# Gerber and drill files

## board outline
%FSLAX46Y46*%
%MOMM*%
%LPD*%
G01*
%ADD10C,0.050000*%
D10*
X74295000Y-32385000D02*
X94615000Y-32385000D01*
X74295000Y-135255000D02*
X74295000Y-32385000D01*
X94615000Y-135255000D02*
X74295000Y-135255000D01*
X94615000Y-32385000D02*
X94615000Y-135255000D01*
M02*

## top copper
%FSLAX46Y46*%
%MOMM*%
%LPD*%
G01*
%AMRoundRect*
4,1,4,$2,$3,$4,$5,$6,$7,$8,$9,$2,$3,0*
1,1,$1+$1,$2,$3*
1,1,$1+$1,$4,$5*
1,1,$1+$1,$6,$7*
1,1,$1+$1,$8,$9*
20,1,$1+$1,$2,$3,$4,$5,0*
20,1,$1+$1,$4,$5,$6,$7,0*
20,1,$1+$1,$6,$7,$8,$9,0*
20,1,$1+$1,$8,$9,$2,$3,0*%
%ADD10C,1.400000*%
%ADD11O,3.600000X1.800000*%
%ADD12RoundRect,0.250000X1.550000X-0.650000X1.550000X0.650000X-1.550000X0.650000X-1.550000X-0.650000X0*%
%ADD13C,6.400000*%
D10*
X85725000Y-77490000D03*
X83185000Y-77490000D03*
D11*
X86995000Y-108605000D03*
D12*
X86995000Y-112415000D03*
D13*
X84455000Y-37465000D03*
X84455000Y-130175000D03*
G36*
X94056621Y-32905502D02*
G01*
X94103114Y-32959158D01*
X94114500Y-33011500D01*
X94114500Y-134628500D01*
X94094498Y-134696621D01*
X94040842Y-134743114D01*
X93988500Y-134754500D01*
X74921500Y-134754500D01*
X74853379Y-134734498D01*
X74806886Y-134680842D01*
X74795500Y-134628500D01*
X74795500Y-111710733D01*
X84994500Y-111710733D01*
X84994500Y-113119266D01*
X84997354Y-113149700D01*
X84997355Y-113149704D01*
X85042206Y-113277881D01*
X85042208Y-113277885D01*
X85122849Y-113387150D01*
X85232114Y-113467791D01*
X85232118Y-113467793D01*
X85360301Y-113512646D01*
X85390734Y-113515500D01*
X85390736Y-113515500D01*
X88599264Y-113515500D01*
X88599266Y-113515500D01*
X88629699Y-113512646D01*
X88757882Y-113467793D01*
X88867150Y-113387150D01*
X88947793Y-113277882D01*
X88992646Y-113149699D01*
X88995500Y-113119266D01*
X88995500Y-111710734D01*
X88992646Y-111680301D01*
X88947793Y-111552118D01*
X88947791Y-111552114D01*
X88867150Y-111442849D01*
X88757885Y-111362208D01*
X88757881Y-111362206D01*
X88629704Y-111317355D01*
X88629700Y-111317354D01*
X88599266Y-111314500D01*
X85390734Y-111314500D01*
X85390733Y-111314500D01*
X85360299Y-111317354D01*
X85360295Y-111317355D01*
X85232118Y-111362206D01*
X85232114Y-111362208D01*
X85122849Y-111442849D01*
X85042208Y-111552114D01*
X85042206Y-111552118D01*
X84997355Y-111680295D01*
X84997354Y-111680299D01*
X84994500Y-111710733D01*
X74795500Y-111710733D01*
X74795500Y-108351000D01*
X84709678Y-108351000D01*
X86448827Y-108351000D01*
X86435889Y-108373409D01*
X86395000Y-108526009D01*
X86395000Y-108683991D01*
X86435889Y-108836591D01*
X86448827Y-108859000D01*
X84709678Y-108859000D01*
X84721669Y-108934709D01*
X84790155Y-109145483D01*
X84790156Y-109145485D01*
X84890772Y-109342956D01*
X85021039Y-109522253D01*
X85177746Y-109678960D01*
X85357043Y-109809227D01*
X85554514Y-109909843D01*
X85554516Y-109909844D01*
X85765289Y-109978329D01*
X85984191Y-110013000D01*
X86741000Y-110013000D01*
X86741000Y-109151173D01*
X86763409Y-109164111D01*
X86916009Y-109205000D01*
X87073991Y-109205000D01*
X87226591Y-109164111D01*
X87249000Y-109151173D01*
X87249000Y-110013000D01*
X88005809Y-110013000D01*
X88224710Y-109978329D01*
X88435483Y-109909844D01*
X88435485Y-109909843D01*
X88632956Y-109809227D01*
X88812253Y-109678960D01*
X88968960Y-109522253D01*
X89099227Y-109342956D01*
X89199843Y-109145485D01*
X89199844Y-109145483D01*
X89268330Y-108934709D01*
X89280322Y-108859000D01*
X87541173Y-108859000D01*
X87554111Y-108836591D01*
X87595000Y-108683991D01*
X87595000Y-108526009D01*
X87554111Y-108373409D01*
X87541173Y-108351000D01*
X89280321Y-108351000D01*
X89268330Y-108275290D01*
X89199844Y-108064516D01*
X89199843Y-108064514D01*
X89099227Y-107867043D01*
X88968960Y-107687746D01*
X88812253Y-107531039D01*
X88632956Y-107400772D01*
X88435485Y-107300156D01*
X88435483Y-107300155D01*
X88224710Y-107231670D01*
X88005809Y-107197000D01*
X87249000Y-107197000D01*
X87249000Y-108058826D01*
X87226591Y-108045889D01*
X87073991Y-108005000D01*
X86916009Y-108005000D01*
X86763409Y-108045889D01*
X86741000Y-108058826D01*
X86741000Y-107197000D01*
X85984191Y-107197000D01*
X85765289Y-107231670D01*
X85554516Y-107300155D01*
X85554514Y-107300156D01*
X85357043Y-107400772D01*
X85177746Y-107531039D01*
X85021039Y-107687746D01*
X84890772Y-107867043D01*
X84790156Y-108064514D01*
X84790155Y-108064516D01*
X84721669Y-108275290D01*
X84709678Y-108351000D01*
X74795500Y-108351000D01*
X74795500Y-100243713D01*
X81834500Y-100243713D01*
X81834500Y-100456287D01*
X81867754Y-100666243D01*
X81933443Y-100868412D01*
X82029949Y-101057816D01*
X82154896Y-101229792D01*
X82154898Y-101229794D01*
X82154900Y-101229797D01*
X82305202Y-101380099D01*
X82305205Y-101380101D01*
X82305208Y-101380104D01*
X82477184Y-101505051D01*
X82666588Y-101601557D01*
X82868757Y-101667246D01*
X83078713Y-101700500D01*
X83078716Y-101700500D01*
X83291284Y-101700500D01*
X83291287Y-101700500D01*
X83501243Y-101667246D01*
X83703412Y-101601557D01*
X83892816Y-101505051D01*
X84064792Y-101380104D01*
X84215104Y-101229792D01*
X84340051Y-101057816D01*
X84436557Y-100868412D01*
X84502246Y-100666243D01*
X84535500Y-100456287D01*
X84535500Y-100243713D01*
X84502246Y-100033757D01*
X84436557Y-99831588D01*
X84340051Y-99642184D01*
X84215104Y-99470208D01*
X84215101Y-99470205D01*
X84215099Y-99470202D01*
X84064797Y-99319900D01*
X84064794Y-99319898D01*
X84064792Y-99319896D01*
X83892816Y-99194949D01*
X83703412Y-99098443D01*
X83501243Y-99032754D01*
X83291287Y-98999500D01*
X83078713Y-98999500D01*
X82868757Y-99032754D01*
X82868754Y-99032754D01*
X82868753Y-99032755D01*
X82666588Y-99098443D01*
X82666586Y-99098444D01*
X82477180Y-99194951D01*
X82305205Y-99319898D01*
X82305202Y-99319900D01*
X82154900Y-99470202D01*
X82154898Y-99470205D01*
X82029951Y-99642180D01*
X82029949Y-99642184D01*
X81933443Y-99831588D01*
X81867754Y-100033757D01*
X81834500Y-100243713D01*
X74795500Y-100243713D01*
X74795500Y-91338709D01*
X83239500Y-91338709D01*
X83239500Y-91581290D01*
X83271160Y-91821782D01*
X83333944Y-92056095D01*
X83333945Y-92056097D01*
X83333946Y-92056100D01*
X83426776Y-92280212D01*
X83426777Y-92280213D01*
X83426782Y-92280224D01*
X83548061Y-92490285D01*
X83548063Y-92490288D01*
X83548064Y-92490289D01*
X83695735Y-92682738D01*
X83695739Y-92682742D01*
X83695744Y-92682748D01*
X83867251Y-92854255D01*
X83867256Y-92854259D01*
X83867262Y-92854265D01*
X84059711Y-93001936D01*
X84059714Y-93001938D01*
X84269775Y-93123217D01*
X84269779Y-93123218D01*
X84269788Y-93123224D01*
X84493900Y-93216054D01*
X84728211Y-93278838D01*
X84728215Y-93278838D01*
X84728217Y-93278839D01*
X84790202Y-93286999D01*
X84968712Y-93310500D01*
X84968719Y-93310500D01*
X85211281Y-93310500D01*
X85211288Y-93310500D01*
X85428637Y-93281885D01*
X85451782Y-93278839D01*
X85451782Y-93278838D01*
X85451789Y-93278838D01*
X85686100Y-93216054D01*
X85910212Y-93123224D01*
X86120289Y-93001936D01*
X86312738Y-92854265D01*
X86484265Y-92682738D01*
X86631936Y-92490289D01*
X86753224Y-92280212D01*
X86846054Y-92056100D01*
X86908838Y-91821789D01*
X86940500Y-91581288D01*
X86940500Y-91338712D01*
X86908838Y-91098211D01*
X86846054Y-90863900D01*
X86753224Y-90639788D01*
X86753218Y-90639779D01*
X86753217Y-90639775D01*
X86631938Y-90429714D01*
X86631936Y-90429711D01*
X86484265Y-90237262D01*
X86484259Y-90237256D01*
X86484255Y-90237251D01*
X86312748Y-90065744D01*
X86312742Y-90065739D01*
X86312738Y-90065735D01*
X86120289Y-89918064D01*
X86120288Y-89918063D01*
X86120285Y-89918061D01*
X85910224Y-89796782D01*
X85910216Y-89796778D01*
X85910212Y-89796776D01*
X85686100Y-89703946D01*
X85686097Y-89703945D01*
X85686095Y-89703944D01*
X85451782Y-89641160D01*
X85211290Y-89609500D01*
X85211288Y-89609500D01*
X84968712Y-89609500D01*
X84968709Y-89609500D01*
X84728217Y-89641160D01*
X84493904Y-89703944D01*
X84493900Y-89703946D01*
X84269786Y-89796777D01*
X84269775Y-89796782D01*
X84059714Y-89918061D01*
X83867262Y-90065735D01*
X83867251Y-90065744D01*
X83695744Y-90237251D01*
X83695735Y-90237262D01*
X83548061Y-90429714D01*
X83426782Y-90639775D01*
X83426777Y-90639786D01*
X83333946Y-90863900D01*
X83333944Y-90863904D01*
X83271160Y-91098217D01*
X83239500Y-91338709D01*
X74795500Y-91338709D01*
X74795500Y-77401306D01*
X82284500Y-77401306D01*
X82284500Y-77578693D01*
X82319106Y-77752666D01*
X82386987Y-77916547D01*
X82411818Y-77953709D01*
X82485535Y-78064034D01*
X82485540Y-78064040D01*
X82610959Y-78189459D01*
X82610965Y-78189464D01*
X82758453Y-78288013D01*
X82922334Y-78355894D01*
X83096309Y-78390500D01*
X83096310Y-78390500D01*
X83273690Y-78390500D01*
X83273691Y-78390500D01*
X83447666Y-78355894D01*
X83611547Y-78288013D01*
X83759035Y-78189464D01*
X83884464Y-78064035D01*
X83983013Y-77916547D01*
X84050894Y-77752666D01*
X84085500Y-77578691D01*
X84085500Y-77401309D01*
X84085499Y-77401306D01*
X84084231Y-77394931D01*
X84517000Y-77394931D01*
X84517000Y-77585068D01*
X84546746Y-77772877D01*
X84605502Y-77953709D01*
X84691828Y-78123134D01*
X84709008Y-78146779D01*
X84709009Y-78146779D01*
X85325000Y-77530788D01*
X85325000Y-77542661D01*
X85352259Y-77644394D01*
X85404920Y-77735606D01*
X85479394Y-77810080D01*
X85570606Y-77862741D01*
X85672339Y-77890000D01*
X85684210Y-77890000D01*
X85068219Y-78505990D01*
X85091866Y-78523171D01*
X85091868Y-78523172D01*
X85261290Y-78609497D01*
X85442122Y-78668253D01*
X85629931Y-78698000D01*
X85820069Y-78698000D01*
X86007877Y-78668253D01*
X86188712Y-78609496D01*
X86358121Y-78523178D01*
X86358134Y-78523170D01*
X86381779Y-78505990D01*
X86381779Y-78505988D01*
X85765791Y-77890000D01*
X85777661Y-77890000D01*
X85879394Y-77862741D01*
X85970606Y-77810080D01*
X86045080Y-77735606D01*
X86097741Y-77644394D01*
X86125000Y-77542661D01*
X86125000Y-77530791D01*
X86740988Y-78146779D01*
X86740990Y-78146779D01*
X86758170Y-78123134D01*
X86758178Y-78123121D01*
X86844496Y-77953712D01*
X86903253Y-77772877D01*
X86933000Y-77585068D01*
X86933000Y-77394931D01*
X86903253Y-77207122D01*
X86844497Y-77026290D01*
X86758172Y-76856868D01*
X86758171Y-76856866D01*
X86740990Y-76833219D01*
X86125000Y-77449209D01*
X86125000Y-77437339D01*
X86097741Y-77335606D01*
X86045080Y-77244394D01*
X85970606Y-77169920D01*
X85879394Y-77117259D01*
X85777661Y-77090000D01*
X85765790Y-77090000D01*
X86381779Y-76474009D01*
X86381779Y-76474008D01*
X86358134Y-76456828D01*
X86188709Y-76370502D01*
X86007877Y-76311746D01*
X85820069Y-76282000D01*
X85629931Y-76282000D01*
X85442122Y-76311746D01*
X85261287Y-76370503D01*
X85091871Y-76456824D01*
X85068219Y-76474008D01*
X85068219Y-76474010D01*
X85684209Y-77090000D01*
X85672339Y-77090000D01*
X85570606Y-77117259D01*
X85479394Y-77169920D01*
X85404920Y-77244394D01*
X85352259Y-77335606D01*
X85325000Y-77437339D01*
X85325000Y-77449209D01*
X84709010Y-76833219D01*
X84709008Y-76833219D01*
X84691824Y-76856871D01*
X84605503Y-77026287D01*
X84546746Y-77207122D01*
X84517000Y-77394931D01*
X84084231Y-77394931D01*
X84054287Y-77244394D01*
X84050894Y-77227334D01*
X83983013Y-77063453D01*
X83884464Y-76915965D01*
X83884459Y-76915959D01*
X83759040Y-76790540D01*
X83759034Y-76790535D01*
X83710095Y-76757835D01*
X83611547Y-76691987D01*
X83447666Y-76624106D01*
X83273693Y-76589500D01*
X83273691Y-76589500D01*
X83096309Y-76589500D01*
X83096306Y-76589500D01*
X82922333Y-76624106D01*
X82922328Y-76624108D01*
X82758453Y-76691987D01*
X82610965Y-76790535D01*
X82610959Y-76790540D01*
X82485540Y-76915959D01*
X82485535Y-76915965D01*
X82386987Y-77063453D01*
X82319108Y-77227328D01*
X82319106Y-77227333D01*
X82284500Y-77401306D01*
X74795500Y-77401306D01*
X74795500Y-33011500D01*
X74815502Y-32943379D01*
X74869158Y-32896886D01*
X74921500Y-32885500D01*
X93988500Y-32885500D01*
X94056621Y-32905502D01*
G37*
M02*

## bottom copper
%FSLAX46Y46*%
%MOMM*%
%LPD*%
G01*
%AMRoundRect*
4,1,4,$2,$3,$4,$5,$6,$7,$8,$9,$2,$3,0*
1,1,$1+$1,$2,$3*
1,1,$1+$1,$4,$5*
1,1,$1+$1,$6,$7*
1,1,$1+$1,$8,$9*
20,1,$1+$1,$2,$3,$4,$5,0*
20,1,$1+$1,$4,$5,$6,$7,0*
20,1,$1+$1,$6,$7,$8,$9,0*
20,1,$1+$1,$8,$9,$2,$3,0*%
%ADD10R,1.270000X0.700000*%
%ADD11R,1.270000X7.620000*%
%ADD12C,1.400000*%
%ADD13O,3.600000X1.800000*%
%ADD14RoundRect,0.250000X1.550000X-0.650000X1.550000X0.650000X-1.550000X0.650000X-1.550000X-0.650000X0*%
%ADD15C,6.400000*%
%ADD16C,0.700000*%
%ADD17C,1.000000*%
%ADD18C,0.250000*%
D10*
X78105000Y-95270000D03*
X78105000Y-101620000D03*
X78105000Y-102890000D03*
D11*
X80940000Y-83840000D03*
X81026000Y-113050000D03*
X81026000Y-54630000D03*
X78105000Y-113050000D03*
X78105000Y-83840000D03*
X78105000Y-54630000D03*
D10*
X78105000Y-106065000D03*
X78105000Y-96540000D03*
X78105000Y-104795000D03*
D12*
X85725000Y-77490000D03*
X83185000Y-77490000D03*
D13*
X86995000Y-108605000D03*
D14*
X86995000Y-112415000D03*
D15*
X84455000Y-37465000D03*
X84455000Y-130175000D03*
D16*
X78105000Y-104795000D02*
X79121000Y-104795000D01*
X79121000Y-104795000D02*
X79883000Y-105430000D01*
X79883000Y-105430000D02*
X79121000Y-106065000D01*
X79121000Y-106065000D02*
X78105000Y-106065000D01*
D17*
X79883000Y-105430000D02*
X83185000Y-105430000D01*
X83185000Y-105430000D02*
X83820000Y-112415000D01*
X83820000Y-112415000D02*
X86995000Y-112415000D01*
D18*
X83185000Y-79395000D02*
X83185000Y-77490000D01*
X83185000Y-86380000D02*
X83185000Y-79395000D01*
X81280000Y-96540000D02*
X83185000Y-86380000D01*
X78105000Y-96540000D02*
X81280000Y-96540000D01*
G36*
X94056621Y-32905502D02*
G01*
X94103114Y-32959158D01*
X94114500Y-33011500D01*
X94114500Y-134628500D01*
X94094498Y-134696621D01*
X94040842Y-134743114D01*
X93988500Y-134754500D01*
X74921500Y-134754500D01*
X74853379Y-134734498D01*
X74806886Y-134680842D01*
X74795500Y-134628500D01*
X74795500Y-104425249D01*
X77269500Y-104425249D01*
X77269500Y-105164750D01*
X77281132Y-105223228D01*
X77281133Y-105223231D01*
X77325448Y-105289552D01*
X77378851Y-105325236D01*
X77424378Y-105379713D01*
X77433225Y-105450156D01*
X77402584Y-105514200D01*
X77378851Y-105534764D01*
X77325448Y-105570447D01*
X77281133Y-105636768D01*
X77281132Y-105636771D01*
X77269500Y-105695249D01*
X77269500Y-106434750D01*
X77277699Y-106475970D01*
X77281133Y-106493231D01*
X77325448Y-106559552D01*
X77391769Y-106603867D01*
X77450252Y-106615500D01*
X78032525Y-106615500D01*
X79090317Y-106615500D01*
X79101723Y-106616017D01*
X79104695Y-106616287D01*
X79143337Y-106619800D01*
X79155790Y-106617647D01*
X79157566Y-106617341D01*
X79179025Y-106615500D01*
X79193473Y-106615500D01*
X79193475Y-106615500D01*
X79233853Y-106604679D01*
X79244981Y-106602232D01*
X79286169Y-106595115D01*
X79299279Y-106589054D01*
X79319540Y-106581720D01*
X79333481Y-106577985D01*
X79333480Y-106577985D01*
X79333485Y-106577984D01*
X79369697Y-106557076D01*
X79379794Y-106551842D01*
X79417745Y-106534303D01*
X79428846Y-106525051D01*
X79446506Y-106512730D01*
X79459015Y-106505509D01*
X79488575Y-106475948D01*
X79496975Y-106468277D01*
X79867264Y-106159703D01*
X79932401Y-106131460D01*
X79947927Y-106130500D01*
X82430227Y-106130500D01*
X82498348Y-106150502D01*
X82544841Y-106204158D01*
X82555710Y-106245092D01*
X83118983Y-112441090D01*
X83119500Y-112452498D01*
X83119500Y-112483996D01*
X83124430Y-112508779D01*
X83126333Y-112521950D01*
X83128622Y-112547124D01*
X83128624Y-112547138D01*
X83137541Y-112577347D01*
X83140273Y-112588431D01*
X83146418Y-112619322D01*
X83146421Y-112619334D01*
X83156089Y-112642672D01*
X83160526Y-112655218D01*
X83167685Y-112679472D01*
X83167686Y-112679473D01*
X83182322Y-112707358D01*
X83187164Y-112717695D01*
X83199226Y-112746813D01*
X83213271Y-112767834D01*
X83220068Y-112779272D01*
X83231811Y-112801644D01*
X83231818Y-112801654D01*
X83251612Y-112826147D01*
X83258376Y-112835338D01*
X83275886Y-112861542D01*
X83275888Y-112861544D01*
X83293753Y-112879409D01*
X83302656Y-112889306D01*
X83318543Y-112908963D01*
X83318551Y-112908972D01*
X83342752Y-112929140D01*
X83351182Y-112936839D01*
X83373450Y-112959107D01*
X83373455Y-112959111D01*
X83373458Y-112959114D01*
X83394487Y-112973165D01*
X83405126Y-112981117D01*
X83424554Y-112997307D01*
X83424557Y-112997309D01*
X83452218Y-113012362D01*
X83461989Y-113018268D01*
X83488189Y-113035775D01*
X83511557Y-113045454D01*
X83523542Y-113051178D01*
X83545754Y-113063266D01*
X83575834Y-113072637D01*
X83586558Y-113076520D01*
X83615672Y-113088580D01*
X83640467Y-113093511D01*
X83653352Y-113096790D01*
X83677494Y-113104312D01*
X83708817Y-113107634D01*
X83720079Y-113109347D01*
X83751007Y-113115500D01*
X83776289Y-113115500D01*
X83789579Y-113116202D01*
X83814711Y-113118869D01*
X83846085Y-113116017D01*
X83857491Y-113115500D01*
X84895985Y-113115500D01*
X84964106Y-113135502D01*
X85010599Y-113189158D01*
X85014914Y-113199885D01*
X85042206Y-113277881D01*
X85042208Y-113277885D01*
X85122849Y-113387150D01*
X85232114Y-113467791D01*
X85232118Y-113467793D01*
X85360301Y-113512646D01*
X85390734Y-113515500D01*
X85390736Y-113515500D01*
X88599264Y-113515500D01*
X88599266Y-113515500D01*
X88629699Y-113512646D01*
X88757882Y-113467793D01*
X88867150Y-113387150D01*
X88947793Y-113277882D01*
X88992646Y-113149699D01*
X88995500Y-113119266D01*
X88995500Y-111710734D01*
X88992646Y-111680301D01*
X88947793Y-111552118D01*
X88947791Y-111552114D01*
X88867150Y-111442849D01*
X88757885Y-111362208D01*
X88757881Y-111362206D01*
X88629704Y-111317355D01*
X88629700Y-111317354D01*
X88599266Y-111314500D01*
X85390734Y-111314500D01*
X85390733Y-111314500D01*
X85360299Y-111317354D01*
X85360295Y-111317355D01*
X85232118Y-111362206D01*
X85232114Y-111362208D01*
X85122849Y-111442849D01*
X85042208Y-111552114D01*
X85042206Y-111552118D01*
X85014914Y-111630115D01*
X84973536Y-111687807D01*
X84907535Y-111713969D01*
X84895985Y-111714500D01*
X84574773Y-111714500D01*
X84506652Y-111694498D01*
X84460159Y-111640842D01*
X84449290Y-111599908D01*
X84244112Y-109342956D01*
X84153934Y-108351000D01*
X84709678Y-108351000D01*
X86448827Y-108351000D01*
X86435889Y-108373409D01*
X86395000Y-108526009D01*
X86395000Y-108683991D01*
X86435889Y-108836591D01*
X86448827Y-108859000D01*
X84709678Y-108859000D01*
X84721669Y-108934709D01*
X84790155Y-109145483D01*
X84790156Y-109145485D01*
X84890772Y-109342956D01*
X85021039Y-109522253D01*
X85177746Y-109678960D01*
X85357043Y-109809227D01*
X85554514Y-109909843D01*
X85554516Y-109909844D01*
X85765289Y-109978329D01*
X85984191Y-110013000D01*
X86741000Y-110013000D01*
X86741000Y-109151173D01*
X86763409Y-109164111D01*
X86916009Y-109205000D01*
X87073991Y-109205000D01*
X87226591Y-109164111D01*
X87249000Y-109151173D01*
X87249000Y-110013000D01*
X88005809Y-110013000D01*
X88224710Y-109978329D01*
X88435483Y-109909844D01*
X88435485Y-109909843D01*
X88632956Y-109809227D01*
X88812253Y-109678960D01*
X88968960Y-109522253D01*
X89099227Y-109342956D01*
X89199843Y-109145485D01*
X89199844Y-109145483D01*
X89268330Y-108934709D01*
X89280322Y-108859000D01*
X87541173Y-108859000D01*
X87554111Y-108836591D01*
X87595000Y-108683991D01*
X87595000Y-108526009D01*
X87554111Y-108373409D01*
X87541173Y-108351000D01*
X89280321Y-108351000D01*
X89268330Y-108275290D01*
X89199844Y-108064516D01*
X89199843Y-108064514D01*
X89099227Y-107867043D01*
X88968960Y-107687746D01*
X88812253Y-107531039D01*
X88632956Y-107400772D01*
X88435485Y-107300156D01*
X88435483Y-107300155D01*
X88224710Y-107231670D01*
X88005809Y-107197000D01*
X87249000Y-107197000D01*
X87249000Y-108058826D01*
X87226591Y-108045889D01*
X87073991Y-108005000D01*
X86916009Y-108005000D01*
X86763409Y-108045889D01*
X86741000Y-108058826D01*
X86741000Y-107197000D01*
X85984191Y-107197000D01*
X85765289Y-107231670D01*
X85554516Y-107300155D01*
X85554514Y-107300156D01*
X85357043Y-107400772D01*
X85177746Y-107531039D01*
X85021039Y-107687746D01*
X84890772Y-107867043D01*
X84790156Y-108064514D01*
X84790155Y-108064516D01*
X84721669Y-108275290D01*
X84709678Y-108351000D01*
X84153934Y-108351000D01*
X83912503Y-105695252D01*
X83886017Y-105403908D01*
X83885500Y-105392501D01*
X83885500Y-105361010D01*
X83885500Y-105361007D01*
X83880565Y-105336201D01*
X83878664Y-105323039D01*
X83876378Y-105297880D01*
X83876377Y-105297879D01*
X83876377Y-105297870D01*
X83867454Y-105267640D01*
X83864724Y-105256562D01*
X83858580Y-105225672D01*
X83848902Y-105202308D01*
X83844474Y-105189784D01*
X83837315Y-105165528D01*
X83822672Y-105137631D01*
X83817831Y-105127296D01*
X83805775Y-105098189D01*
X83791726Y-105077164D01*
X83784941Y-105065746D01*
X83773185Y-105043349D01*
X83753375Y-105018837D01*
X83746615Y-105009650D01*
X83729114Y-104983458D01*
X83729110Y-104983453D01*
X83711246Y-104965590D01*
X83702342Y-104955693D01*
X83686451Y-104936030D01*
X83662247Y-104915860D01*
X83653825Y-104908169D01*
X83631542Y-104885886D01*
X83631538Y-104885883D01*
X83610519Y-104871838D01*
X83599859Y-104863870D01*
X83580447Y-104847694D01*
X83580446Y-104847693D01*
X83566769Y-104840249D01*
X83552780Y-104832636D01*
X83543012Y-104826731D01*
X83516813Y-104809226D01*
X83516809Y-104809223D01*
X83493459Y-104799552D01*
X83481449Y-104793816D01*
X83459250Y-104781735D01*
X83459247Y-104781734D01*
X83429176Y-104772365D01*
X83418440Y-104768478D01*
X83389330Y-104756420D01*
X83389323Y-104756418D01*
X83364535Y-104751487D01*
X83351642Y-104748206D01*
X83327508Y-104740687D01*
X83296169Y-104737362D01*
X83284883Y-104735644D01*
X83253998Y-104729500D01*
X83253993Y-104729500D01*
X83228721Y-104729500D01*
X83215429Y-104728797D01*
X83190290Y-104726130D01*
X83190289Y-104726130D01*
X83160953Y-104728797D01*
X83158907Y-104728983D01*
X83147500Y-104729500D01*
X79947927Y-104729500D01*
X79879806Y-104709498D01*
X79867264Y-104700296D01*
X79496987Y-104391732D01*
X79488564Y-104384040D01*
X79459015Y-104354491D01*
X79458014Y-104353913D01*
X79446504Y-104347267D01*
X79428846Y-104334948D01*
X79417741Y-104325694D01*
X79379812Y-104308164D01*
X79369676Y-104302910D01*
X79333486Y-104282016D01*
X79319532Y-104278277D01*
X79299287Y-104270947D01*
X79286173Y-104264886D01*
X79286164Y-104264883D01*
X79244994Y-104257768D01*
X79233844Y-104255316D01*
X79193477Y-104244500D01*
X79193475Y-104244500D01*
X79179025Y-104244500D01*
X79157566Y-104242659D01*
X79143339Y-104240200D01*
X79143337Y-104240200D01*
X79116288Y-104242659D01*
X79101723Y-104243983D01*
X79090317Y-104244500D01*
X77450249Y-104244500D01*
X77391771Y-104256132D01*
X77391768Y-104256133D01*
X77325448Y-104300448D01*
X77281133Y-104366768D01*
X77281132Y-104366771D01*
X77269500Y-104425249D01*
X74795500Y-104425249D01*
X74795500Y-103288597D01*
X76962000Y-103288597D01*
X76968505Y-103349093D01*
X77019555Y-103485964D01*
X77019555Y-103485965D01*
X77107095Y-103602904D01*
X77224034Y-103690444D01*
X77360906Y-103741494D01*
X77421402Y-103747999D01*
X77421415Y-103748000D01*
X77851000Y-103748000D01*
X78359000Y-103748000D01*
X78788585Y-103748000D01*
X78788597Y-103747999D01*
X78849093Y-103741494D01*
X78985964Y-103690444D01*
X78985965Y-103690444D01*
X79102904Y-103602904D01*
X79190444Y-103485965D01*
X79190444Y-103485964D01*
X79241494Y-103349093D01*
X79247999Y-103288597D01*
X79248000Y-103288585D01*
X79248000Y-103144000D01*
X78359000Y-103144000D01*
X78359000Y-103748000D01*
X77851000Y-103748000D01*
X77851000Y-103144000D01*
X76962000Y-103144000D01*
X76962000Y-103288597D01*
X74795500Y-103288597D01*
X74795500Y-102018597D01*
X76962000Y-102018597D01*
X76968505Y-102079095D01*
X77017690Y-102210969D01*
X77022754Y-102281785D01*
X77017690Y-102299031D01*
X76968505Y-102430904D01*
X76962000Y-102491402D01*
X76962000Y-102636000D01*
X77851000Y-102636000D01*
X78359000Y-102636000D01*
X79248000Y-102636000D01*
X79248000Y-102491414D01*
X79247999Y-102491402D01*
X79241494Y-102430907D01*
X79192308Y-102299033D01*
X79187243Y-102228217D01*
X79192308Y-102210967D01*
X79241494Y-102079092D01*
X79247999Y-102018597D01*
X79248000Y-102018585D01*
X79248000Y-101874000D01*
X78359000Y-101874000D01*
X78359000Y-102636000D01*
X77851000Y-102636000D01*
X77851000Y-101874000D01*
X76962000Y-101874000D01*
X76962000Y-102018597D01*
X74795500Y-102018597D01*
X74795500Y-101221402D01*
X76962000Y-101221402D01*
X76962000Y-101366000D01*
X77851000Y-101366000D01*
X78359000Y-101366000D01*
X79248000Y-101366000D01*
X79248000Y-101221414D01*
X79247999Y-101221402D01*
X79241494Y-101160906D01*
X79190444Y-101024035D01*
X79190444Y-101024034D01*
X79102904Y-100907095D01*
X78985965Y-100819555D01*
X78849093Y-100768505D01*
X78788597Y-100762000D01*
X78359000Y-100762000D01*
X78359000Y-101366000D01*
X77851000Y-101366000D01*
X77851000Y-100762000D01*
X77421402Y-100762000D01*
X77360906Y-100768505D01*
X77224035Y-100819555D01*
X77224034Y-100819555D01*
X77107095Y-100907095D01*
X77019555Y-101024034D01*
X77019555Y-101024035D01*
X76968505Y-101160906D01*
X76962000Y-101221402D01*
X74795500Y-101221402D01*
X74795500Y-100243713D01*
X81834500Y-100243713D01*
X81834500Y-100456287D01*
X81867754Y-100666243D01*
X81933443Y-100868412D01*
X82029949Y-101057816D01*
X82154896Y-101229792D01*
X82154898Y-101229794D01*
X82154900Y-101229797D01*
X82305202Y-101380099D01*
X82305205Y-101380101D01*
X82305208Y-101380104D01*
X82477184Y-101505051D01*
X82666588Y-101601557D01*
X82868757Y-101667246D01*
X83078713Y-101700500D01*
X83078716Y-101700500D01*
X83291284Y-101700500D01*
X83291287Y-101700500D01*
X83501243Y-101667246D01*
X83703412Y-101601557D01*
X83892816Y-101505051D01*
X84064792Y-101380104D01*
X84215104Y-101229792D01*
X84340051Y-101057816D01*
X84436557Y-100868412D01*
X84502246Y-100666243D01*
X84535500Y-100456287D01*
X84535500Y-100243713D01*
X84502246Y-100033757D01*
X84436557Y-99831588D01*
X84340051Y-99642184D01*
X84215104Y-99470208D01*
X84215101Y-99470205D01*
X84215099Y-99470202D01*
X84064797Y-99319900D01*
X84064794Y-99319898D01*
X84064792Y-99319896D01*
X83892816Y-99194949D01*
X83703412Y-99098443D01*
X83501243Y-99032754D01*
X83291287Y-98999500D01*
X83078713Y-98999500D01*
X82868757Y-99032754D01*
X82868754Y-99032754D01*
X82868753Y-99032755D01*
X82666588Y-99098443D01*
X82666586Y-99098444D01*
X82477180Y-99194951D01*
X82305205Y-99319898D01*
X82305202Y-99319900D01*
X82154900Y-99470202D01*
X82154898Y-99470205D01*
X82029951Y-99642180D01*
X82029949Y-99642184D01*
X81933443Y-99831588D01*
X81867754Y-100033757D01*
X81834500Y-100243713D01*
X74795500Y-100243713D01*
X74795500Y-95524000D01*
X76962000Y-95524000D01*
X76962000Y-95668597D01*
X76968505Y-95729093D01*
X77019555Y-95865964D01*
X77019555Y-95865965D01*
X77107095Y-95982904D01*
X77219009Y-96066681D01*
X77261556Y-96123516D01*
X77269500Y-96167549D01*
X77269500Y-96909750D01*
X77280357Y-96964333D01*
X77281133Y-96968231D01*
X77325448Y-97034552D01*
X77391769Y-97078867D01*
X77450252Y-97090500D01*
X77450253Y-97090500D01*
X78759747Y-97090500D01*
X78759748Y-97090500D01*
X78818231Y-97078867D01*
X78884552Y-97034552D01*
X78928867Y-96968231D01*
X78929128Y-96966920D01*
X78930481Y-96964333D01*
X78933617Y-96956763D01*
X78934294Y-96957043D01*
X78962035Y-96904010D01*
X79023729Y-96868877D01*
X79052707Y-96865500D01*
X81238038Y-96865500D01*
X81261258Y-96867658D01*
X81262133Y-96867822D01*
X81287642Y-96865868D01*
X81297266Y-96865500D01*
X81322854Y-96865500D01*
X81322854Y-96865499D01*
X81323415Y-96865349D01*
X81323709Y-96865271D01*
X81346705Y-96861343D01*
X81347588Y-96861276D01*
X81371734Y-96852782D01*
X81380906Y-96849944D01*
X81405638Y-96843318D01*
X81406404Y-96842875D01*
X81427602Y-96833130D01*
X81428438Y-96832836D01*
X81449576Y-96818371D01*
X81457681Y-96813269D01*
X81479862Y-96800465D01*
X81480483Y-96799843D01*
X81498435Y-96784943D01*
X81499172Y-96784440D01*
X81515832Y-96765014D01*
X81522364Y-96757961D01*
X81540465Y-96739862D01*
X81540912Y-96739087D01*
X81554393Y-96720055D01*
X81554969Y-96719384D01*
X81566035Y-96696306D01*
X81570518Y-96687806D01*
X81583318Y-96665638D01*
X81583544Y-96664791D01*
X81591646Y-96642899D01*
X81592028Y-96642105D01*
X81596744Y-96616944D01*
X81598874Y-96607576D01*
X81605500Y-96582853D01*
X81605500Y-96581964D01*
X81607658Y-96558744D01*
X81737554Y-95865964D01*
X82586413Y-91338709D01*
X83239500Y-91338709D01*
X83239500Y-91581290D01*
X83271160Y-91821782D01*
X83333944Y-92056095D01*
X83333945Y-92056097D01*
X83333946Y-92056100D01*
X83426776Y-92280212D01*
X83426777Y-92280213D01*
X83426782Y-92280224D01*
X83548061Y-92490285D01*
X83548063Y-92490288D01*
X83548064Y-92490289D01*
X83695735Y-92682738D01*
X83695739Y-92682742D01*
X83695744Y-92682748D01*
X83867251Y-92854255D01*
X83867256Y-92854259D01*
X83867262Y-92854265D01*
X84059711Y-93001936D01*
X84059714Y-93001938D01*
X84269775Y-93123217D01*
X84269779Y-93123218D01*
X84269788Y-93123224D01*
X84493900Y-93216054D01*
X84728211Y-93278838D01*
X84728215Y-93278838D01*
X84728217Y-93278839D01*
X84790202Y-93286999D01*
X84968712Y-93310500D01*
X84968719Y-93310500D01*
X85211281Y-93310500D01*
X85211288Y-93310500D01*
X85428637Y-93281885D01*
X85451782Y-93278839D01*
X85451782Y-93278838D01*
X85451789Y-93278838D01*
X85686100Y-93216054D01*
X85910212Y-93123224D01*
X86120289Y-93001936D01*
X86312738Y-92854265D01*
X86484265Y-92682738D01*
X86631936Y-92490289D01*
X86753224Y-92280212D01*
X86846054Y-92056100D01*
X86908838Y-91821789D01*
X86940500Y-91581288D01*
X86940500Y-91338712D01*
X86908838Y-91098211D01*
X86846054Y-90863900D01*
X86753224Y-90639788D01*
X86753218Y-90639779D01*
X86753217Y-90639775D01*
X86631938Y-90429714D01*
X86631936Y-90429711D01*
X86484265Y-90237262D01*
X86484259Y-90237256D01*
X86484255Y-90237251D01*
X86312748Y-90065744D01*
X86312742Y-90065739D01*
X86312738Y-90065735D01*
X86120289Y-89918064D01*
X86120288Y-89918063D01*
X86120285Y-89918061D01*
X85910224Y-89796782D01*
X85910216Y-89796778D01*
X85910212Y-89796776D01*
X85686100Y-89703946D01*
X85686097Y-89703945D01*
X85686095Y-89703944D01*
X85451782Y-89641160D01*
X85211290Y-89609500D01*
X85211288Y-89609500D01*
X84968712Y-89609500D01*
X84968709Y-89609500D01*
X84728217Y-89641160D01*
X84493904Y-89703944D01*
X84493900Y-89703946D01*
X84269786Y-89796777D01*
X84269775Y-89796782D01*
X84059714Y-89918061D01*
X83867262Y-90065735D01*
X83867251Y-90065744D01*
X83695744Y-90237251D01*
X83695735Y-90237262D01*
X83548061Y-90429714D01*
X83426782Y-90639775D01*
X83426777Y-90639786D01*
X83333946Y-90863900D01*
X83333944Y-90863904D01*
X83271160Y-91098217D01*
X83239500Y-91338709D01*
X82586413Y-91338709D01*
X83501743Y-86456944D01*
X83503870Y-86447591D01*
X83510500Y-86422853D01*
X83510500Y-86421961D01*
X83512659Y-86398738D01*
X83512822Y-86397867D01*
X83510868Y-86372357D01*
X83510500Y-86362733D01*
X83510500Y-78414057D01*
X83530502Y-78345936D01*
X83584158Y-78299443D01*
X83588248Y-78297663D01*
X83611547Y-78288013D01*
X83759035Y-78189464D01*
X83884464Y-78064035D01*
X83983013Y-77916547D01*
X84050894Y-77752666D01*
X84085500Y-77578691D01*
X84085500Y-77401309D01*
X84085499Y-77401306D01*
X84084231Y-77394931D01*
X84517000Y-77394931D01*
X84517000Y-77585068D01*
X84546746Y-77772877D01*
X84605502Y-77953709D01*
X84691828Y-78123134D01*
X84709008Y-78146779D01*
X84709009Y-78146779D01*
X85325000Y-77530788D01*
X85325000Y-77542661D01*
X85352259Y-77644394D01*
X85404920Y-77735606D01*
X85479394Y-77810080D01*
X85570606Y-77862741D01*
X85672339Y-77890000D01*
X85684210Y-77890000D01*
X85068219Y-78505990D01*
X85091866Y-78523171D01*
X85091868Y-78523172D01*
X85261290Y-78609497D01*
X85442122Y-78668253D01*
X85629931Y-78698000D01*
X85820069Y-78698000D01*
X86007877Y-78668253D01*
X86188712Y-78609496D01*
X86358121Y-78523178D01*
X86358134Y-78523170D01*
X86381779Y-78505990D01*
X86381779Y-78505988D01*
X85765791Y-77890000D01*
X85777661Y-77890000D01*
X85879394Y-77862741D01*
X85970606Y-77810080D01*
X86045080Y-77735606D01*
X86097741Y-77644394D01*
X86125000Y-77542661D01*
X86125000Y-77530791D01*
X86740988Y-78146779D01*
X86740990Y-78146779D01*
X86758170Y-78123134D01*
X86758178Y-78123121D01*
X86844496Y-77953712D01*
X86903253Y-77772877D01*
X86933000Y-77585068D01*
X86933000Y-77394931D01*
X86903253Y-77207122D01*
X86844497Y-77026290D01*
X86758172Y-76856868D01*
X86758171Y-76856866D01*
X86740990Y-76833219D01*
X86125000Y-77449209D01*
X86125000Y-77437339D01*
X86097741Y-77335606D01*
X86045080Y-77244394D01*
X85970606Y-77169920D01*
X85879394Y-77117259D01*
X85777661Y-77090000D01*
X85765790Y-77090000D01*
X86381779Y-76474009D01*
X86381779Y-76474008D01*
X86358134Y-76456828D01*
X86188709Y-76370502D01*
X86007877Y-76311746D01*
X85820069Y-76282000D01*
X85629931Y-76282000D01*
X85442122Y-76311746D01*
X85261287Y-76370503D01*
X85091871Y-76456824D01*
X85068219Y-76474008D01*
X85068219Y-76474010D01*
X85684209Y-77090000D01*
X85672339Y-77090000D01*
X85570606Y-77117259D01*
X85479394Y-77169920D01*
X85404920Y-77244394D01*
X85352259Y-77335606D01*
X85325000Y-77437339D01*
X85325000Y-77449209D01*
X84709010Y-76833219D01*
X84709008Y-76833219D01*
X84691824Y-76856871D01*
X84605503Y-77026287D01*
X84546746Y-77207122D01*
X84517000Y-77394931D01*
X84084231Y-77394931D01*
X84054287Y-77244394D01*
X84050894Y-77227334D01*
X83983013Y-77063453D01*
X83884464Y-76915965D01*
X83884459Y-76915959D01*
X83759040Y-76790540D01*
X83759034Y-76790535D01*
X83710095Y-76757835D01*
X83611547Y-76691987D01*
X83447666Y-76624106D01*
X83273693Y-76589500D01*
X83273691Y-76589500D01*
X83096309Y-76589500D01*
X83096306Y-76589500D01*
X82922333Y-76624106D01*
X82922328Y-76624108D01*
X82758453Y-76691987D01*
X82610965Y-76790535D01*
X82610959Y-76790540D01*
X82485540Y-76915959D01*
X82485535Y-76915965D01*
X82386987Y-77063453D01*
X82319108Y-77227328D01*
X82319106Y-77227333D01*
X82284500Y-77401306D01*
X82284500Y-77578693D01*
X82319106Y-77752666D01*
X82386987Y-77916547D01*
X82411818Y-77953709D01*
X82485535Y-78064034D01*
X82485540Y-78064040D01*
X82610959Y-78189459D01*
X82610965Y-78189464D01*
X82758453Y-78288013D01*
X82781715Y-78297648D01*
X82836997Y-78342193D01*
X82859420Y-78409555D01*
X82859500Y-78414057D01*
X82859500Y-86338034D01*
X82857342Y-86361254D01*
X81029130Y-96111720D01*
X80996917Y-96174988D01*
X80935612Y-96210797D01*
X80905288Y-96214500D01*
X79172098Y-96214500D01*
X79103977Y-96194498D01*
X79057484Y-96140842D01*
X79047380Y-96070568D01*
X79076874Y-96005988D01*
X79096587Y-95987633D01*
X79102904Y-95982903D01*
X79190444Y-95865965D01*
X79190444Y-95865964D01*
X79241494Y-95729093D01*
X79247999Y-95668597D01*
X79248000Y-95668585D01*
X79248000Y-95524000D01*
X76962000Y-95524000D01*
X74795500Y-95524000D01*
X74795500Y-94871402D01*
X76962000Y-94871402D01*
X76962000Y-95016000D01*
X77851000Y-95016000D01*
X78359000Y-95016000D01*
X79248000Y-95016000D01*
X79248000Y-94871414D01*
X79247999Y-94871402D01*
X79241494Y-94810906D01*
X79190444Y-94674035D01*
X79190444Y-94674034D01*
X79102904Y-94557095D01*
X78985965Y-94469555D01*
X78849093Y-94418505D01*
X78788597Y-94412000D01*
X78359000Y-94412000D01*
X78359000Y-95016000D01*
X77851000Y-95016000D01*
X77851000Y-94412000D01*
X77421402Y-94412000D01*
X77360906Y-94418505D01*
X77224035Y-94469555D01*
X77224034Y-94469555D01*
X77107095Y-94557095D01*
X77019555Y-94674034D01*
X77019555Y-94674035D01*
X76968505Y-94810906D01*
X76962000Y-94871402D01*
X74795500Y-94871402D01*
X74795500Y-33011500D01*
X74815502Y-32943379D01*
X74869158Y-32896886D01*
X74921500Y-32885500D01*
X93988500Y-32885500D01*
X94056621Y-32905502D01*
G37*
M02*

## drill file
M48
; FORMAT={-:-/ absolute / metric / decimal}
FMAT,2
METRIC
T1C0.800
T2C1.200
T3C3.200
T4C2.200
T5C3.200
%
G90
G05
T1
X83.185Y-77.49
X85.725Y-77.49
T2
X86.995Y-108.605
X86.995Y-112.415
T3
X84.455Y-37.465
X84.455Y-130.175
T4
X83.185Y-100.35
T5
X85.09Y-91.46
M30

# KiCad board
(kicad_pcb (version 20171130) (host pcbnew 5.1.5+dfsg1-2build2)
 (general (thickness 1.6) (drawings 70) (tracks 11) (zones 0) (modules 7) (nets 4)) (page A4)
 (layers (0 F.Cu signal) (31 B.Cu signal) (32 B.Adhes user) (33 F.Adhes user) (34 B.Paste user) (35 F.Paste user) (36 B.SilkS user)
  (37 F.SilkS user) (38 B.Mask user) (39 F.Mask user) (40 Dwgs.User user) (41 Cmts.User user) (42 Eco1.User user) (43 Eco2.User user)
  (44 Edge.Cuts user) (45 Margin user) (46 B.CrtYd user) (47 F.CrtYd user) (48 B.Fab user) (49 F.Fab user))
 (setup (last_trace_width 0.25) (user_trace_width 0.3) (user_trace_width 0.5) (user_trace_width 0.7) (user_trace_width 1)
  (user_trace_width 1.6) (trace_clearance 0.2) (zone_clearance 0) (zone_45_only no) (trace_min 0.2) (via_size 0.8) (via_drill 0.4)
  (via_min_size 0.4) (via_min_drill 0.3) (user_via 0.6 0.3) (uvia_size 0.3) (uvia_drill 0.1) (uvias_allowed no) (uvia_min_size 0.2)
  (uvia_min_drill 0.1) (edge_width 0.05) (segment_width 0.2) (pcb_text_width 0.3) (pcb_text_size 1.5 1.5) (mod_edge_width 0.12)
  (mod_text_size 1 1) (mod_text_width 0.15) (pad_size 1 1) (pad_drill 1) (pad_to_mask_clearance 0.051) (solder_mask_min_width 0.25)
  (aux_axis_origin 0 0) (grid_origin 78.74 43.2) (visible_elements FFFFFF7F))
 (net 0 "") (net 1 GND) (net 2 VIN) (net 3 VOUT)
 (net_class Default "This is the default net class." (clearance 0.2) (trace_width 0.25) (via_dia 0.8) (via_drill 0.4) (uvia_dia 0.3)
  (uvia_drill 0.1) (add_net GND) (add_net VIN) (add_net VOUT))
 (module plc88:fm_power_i (layer F.Cu) (at 80.645 55.265)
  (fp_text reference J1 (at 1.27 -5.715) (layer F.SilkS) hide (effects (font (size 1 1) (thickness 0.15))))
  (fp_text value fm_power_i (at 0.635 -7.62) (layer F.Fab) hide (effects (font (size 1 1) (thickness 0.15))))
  (pad 4 smd rect (at -2.54 40.005) (size 1.27 0.7) (layers B.Cu B.Paste B.Mask) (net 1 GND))
  (pad 2 smd rect (at -2.54 46.355) (size 1.27 0.7) (layers B.Cu B.Paste B.Mask) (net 1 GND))
  (pad 2 smd rect (at -2.54 47.625) (size 1.27 0.7) (layers B.Cu B.Paste B.Mask) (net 1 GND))
  (pad 5 smd rect (at 0.295 28.575) (size 1.27 7.62) (layers B.Cu B.Paste B.Mask) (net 1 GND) (zone_connect 2))
  (pad 5 smd rect (at 0.381 57.785) (size 1.27 7.62) (layers B.Cu B.Paste B.Mask) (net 1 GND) (zone_connect 2))
  (pad 5 smd rect (at 0.381 -0.635) (size 1.27 7.62) (layers B.Cu B.Paste B.Mask) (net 1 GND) (zone_connect 2))
  (pad 5 smd rect (at -2.54 57.785) (size 1.27 7.62) (layers B.Cu B.Paste B.Mask) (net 1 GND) (zone_connect 2))
  (pad 5 smd rect (at -2.54 28.575) (size 1.27 7.62) (layers B.Cu B.Paste B.Mask) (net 1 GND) (zone_connect 2))
  (pad 5 smd rect (at -2.54 -0.635) (size 1.27 7.62) (layers B.Cu B.Paste B.Mask) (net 1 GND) (zone_connect 2))
  (pad 1 smd rect (at -2.54 50.8) (size 1.27 0.7) (layers B.Cu B.Paste B.Mask) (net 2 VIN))
  (pad 3 smd rect (at -2.54 41.275) (size 1.27 0.7) (layers B.Cu B.Paste B.Mask) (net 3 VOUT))
  (pad 1 smd rect (at -2.54 49.53) (size 1.27 0.7) (layers B.Cu B.Paste B.Mask) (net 2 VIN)))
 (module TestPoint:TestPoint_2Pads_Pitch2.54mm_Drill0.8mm (layer F.Cu) (at 83.185 77.49)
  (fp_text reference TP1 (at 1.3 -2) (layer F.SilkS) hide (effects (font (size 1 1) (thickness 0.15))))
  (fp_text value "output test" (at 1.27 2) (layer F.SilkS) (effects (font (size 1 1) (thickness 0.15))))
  (pad 2 thru_hole circle (at 2.54 0) (size 1.4 1.4) (drill 0.8) (layers *.Cu *.Mask) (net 1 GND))
  (pad 1 thru_hole circle (at 0 0) (size 1.4 1.4) (drill 0.8) (layers *.Cu *.Mask) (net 3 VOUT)))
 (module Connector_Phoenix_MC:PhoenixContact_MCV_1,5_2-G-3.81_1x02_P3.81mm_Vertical (layer F.Cu) (at 86.995 112.415 90)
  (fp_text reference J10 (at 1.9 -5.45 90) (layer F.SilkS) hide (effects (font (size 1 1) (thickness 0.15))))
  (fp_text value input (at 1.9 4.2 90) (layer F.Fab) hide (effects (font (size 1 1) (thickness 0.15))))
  (pad 2 thru_hole oval (at 3.81 0 90) (size 1.8 3.6) (drill 1.2) (layers *.Cu *.Mask) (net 1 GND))
  (pad 1 thru_hole roundrect (at 0 0 90) (size 1.8 3.6) (drill 1.2) (layers *.Cu *.Mask) (roundrect_rratio 0.138889) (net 2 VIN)))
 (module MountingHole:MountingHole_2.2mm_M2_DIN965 (layer F.Cu) (at 83.185 100.35)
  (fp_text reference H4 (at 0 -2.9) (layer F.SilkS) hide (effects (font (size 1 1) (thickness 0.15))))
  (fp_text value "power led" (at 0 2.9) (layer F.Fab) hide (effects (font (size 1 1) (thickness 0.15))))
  (pad 1 np_thru_hole circle (at 0 0) (size 2.2 2.2) (drill 2.2) (layers *.Cu *.Mask)))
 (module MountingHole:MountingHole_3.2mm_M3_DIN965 (layer F.Cu) (at 85.09 91.46)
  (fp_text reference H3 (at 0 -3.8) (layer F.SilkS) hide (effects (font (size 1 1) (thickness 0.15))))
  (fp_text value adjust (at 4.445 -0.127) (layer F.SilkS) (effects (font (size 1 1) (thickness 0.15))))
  (pad 1 np_thru_hole circle (at 0 0) (size 3.2 3.2) (drill 3.2) (layers *.Cu *.Mask)))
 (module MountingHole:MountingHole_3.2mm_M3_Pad (layer F.Cu) (at 84.455 37.465)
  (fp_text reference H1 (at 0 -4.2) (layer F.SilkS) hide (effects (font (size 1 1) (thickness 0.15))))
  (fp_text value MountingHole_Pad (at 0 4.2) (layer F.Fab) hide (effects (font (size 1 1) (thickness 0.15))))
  (pad 1 thru_hole circle (at 0 0) (size 6.4 6.4) (drill 3.2) (layers *.Cu *.Mask) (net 1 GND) (zone_connect 2)))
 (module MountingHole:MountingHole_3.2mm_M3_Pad (layer F.Cu) (at 84.455 130.175)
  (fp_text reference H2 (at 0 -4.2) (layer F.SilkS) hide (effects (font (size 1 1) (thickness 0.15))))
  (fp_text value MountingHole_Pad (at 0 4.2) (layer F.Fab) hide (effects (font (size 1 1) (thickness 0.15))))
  (pad 1 thru_hole circle (at 0 0) (size 6.4 6.4) (drill 3.2) (layers *.Cu *.Mask) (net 1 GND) (zone_connect 2)))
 (gr_line (start 74.295 32.385) (end 94.615 32.385) (layer Edge.Cuts) (width 0.05))
 (gr_line (start 74.295 135.255) (end 74.295 32.385) (layer Edge.Cuts) (width 0.05))
 (gr_line (start 94.615 135.255) (end 74.295 135.255) (layer Edge.Cuts) (width 0.05))
 (gr_line (start 94.615 32.385) (end 94.615 135.255) (layer Edge.Cuts) (width 0.05))
 (segment (start 78.105 104.795) (end 79.121 104.795) (width 0.7) (layer B.Cu) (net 2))
 (segment (start 79.121 104.795) (end 79.883 105.43) (width 0.7) (layer B.Cu) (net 2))
 (segment (start 79.883 105.43) (end 79.121 106.065) (width 0.7) (layer B.Cu) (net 2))
 (segment (start 79.121 106.065) (end 78.105 106.065) (width 0.7) (layer B.Cu) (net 2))
 (segment (start 79.883 105.43) (end 83.185 105.43) (width 1) (layer B.Cu) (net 2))
 (segment (start 83.185 105.43) (end 83.82 112.415) (width 1) (layer B.Cu) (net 2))
 (segment (start 83.82 112.415) (end 86.995 112.415) (width 1) (layer B.Cu) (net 2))
 (segment (start 83.185 79.395) (end 83.185 77.49) (width 0.25) (layer B.Cu) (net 3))
 (segment (start 83.185 86.38) (end 83.185 79.395) (width 0.25) (layer B.Cu) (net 3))
 (segment (start 81.28 96.54) (end 83.185 86.38) (width 0.25) (layer B.Cu) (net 3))
 (segment (start 78.105 96.54) (end 81.28 96.54) (width 0.25) (layer B.Cu) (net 3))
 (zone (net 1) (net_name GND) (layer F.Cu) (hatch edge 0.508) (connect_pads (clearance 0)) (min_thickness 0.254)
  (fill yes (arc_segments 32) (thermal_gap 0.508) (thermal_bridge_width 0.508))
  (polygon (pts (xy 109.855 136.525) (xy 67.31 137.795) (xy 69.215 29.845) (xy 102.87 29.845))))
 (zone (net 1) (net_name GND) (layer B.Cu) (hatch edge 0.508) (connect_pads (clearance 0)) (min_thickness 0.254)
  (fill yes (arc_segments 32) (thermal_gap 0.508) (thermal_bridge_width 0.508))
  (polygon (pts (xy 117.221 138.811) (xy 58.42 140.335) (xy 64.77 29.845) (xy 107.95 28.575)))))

